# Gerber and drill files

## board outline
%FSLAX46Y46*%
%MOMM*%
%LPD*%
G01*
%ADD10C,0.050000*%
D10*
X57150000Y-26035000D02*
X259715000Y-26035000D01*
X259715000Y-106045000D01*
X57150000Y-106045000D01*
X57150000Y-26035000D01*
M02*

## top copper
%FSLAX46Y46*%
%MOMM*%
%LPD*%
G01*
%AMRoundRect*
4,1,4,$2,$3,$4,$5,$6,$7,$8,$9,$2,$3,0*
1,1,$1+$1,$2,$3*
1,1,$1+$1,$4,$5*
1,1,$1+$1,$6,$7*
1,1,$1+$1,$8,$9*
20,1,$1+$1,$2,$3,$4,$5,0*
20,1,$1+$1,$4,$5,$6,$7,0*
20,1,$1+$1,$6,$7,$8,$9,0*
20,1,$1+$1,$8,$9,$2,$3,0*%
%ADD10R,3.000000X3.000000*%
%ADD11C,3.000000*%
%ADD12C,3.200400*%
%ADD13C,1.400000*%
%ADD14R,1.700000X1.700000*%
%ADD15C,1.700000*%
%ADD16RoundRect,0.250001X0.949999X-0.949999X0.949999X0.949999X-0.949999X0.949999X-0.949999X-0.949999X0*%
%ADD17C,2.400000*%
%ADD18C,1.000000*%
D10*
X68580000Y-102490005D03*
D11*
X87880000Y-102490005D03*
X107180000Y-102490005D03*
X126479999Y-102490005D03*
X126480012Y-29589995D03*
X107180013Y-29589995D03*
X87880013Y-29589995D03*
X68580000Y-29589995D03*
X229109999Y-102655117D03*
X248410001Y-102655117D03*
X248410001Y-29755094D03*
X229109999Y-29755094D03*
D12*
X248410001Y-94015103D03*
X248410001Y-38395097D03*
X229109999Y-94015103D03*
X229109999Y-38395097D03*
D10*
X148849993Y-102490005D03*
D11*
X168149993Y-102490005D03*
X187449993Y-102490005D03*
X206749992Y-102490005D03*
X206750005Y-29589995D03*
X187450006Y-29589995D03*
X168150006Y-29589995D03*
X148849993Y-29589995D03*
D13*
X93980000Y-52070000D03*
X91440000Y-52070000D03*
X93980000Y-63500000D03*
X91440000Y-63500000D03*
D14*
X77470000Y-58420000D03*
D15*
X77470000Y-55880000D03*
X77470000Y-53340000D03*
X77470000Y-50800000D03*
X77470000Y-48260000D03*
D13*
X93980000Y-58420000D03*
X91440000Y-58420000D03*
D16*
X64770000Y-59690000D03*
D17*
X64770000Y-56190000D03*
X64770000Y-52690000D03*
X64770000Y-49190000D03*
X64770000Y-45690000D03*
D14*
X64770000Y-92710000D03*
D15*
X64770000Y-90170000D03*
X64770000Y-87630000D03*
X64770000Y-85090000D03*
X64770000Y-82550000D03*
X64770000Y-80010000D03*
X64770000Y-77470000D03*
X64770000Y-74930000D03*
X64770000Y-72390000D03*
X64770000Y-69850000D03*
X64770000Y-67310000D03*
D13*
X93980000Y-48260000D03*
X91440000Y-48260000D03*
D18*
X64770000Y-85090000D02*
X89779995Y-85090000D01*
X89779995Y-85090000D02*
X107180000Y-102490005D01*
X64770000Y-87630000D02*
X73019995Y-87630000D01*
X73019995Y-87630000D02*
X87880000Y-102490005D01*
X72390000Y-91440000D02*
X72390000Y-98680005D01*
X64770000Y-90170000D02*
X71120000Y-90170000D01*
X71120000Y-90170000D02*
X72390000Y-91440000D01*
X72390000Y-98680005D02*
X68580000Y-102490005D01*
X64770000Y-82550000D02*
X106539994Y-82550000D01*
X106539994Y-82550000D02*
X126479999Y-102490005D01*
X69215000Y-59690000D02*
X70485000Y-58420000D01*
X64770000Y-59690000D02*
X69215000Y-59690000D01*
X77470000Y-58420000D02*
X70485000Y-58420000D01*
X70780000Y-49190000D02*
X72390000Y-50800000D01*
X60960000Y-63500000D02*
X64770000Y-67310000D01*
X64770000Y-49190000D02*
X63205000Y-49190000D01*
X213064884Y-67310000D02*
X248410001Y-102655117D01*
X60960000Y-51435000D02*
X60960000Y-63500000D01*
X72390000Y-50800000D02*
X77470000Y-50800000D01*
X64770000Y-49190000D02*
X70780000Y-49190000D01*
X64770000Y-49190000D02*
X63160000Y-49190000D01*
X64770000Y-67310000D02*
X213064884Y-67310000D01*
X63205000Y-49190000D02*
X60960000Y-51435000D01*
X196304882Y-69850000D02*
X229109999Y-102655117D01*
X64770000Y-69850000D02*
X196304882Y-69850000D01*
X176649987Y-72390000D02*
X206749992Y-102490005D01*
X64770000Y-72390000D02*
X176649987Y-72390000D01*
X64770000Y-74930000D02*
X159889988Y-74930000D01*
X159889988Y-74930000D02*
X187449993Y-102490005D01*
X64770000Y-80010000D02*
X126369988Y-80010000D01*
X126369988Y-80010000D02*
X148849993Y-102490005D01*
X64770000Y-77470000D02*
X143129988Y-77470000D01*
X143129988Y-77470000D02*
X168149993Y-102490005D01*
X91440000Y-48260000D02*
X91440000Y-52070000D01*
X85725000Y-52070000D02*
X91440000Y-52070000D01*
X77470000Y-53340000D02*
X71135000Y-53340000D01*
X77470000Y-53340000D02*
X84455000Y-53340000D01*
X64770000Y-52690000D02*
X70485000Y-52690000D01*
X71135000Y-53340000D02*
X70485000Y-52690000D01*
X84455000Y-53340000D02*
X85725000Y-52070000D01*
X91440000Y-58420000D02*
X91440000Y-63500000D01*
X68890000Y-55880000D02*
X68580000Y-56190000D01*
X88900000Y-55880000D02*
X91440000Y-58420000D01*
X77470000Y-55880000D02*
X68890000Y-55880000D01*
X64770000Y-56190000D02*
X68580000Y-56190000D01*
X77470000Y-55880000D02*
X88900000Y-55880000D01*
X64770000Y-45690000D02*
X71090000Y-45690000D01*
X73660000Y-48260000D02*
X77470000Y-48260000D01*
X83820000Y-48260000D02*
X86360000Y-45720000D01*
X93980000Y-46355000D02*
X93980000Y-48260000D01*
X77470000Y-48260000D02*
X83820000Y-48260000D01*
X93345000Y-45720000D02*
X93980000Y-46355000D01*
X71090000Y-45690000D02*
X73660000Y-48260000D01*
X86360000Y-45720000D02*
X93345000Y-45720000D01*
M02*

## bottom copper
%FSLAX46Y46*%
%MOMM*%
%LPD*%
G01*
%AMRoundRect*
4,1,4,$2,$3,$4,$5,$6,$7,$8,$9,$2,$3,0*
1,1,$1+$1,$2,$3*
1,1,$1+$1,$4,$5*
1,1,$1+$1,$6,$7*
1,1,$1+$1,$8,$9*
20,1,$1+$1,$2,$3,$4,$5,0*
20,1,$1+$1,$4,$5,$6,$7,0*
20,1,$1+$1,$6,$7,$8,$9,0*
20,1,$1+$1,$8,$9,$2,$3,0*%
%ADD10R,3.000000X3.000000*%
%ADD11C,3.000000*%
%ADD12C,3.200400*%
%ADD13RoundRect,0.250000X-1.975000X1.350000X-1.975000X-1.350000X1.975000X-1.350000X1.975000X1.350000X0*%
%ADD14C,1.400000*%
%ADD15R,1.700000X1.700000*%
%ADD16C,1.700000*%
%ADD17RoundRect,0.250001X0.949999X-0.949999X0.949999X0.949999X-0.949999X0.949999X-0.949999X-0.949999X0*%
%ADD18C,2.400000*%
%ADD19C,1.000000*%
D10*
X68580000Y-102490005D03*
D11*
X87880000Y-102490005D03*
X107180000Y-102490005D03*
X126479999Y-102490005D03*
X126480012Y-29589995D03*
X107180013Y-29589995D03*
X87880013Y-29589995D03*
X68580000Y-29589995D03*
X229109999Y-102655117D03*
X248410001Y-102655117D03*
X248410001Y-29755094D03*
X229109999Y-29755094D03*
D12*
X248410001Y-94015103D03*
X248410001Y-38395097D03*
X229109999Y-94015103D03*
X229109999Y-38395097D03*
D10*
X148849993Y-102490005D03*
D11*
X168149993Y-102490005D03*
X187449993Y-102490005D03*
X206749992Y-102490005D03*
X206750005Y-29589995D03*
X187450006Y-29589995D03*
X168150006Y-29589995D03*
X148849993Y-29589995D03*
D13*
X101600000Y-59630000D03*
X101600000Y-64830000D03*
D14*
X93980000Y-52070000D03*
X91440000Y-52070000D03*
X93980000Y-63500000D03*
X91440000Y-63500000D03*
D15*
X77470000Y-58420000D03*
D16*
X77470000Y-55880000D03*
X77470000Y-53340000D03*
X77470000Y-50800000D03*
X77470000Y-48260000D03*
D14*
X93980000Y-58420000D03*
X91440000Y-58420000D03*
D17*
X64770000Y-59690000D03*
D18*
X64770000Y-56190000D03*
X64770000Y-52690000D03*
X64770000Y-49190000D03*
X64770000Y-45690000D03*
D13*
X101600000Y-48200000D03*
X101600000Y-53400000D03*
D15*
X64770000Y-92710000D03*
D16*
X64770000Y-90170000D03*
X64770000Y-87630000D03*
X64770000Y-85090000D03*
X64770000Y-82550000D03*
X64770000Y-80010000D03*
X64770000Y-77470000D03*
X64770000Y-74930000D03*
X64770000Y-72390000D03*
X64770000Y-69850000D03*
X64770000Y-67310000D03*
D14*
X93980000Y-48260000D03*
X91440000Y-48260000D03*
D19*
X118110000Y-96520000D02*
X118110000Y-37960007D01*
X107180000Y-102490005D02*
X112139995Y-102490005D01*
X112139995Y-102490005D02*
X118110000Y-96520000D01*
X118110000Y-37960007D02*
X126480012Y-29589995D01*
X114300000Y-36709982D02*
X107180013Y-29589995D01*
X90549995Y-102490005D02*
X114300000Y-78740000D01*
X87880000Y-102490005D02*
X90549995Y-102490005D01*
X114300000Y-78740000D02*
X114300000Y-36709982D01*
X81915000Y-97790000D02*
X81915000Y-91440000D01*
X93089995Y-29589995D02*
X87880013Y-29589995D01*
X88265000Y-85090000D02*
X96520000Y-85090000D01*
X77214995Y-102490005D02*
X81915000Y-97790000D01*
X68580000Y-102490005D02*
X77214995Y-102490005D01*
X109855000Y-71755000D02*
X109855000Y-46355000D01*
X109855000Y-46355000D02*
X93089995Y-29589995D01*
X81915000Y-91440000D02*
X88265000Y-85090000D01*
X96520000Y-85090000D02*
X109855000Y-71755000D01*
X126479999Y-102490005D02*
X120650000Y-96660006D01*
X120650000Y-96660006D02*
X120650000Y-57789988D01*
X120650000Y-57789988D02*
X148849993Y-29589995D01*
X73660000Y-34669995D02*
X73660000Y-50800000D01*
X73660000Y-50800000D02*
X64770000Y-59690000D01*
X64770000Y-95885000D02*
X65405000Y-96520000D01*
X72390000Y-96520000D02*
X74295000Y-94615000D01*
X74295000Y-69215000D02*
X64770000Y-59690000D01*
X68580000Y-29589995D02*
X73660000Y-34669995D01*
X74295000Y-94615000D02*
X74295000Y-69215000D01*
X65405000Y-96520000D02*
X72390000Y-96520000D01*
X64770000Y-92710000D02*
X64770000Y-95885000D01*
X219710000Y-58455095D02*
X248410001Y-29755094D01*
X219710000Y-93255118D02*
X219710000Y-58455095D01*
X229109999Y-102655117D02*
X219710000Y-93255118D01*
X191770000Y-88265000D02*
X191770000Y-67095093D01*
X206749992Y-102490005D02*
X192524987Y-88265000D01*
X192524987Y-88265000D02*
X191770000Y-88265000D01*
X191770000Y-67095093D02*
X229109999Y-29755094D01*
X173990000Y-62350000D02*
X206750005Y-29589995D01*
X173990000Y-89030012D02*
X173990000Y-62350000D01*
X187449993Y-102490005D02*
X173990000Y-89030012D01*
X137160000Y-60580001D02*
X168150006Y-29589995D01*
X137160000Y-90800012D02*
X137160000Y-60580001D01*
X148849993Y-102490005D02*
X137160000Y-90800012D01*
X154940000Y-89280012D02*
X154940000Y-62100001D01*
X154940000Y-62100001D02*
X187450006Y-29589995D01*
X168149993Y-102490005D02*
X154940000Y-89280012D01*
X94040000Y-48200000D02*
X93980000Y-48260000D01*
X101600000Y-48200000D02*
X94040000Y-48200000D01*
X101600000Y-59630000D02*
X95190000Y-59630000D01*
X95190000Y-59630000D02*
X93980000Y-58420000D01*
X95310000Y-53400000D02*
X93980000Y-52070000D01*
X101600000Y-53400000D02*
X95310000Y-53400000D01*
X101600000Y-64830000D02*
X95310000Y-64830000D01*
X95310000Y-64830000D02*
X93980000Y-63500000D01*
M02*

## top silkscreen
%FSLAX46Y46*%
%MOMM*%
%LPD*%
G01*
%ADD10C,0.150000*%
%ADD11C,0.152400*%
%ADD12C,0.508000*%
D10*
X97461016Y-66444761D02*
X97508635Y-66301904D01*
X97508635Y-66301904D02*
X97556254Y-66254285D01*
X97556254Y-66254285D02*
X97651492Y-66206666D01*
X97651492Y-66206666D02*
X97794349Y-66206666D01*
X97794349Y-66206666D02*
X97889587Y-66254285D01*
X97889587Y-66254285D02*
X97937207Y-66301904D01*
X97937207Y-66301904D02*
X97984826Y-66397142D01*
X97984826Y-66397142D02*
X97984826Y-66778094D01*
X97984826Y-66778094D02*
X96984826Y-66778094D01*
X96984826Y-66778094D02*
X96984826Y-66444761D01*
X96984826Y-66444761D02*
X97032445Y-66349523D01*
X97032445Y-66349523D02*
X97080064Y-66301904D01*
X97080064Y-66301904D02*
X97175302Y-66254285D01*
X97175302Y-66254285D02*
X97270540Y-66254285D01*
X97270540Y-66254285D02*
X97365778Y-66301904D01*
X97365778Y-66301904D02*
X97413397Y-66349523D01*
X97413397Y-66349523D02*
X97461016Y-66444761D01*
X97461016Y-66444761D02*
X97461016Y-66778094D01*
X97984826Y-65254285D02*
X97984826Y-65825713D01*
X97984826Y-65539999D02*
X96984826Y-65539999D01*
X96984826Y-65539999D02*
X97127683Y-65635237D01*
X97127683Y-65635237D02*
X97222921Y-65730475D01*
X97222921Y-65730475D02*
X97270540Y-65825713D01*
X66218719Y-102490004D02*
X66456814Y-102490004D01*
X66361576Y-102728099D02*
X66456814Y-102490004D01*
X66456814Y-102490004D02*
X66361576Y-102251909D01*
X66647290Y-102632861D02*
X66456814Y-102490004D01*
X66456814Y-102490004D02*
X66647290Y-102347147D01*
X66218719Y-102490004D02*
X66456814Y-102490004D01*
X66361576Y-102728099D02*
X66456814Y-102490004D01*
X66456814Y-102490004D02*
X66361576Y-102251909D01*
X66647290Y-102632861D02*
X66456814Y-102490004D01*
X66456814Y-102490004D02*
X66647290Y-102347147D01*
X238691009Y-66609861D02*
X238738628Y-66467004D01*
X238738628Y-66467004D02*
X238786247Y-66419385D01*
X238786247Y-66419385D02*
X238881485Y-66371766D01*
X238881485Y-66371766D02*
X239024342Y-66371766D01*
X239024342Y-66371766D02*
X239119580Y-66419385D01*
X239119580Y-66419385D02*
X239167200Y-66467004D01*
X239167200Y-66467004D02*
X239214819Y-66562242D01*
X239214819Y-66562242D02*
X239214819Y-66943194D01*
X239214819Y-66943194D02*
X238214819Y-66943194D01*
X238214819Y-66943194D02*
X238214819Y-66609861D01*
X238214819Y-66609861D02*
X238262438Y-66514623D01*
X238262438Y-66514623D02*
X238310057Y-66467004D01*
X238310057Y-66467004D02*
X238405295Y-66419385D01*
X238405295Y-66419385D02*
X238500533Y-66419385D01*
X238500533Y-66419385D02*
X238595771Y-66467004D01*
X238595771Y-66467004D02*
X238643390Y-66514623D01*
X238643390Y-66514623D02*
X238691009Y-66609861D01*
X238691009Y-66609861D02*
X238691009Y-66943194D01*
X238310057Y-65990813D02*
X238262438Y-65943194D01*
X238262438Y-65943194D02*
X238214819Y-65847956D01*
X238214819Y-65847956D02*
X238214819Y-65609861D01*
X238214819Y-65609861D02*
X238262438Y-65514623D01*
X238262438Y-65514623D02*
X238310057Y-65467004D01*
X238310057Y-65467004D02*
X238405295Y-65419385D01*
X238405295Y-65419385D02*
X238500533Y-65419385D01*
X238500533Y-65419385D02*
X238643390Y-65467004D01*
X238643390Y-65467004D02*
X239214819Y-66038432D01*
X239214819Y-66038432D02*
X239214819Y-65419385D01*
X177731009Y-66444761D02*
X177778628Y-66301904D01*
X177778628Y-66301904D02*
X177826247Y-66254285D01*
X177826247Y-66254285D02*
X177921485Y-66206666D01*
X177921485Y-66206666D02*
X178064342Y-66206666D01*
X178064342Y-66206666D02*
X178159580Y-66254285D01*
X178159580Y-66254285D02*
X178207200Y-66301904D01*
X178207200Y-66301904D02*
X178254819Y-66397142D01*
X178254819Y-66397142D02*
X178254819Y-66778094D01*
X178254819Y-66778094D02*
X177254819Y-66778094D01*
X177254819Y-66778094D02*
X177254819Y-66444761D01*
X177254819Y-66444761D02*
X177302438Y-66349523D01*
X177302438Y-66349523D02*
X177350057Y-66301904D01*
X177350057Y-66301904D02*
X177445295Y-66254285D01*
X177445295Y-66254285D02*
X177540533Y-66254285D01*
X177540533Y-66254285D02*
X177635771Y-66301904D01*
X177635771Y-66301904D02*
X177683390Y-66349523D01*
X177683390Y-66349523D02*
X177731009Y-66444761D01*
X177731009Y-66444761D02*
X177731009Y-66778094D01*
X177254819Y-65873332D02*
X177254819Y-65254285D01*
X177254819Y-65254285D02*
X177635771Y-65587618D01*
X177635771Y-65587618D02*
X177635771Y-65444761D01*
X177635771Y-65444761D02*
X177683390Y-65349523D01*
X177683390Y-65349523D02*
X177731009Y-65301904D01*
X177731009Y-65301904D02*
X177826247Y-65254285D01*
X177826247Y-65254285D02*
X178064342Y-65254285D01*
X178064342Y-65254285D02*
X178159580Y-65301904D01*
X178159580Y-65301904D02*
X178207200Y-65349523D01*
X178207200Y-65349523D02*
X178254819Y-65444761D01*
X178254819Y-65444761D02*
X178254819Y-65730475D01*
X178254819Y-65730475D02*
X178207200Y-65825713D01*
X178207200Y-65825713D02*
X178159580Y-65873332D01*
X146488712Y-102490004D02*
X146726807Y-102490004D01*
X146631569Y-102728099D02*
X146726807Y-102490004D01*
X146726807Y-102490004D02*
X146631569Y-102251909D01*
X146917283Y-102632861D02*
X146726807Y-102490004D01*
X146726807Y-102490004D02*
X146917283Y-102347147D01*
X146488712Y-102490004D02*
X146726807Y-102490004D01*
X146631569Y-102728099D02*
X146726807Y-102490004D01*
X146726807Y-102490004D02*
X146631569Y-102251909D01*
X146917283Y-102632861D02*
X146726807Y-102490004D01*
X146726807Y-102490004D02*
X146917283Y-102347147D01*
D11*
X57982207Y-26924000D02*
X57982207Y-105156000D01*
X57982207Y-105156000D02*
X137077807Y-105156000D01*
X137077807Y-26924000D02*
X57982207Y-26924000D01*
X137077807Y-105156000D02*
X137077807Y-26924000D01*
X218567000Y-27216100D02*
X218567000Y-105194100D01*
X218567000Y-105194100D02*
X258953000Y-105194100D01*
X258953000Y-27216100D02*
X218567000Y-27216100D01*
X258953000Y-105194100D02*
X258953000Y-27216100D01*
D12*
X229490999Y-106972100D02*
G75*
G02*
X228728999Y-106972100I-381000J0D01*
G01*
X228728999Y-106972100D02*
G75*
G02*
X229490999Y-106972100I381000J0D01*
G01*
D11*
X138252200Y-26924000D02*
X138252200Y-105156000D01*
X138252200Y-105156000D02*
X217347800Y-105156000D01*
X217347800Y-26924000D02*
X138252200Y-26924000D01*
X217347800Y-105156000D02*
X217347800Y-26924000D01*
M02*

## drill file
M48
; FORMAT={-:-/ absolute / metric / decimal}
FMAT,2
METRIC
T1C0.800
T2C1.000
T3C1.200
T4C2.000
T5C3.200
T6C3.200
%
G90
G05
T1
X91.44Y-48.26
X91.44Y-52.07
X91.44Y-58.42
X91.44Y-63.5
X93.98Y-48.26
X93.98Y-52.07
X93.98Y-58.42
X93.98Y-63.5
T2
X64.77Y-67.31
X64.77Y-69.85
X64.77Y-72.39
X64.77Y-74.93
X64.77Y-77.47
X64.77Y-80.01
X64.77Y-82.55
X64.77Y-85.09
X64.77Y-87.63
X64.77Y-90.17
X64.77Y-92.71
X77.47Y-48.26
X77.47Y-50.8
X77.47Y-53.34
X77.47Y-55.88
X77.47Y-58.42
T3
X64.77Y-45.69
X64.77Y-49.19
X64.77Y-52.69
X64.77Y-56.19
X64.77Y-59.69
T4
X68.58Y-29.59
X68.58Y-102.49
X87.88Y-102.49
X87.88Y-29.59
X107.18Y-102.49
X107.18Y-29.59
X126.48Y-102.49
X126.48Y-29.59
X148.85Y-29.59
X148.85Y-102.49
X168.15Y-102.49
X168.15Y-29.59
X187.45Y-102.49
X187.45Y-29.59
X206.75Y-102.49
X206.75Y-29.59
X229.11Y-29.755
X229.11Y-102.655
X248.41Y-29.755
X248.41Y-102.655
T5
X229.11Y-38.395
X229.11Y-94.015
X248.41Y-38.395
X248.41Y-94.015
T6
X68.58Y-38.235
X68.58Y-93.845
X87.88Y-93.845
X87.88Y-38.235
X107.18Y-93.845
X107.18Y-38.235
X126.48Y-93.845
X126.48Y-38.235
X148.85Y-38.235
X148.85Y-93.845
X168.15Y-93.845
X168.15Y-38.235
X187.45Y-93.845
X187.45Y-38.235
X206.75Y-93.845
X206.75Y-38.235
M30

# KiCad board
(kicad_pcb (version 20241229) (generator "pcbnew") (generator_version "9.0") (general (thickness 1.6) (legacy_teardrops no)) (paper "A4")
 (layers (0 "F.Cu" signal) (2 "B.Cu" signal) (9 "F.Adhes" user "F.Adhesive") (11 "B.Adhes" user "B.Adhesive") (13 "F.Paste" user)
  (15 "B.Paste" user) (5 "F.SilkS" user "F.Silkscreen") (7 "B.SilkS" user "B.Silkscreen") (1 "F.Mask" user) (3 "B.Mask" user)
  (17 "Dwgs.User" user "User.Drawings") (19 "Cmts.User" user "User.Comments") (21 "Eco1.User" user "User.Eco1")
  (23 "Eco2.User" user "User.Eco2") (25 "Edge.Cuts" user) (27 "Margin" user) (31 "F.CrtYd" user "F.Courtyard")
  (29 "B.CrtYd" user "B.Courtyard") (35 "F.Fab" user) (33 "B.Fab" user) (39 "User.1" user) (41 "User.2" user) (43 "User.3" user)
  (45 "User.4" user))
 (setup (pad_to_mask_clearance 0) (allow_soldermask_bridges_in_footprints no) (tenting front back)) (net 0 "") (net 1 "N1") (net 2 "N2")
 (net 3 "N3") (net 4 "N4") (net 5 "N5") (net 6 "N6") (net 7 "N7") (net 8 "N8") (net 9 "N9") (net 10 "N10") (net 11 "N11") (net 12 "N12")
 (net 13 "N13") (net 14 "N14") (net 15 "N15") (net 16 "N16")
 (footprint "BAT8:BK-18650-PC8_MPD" (layer "F.Cu") (at 68.58 102.490005 90)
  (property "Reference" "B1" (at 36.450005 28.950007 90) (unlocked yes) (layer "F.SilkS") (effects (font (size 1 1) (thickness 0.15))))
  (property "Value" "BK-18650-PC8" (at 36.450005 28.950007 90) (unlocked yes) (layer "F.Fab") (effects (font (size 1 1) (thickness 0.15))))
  (fp_line (start 75.566005 -10.597793) (end -2.665995 -10.597793) (stroke (width 0.1524) (type solid)) (layer "F.SilkS"))
  (fp_line (start -2.665995 -10.597793) (end -2.665995 68.497807) (stroke (width 0.1524) (type solid)) (layer "F.SilkS"))
  (fp_line (start 75.566005 68.497807) (end 75.566005 -10.597793) (stroke (width 0.1524) (type solid)) (layer "F.SilkS"))
  (fp_line (start -2.665995 68.497807) (end 75.566005 68.497807) (stroke (width 0.1524) (type solid)) (layer "F.SilkS"))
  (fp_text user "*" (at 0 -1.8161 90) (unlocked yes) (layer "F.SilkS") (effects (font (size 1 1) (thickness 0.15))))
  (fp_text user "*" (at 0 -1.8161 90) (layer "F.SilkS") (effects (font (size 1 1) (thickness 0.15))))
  (pad "" np_thru_hole circle (at 8.644999 0 90) (size 3.2004 3.2004) (drill 3.2004) (layers))
  (pad "" np_thru_hole circle (at 8.644999 19.3 90) (size 3.2004 3.2004) (drill 3.2004) (layers))
  (pad "" np_thru_hole circle (at 8.644999 38.6 90) (size 3.2004 3.2004) (drill 3.2004) (layers))
  (pad "" np_thru_hole circle (at 8.644999 57.899999 90) (size 3.2004 3.2004) (drill 3.2004) (layers))
  (pad "" np_thru_hole circle (at 64.25501 0 90) (size 3.2004 3.2004) (drill 3.2004) (layers))
  (pad "" np_thru_hole circle (at 64.25501 19.300013 90) (size 3.2004 3.2004) (drill 3.2004) (layers))
  (pad "" np_thru_hole circle (at 64.25501 38.600013 90) (size 3.2004 3.2004) (drill 3.2004) (layers))
  (pad "" np_thru_hole circle (at 64.25501 57.900012 90) (size 3.2004 3.2004) (drill 3.2004) (layers))
  (pad "1" thru_hole rect (at 0 0 90) (size 3 3) (drill 2) (layers "*.Cu" "*.Mask") (remove_unused_layers no) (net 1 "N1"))
  (pad "2" thru_hole circle (at 0 19.3 90) (size 3 3) (drill 2) (layers "*.Cu" "*.Mask") (remove_unused_layers no) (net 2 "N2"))
  (pad "3" thru_hole circle (at 0 38.6 90) (size 3 3) (drill 2) (layers "*.Cu" "*.Mask") (remove_unused_layers no) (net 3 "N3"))
  (pad "4" thru_hole circle (at 0 57.899999 90) (size 3 3) (drill 2) (layers "*.Cu" "*.Mask") (remove_unused_layers no) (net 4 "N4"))
  (pad "5" thru_hole circle (at 72.90001 57.900012 90) (size 3 3) (drill 2) (layers "*.Cu" "*.Mask") (remove_unused_layers no) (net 3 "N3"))
  (pad "6" thru_hole circle (at 72.90001 38.600013 90) (size 3 3) (drill 2) (layers "*.Cu" "*.Mask") (remove_unused_layers no) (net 2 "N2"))
  (pad "7" thru_hole circle (at 72.90001 19.300013 90) (size 3 3) (drill 2) (layers "*.Cu" "*.Mask") (remove_unused_layers no) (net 1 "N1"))
  (pad "8" thru_hole circle (at 72.90001 0 90) (size 3 3) (drill 2) (layers "*.Cu" "*.Mask") (remove_unused_layers no) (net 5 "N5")))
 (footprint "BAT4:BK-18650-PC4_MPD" (layer "F.Cu") (at 229.109999 102.655117 90)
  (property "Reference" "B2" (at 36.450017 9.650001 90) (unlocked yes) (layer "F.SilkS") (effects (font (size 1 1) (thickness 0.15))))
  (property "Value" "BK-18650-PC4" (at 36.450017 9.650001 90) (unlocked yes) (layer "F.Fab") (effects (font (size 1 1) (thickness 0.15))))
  (fp_line (start 75.439017 -10.542999) (end -2.538983 -10.542999) (stroke (width 0.1524) (type solid)) (layer "F.SilkS"))
  (fp_line (start -2.538983 -10.542999) (end -2.538983 29.843001) (stroke (width 0.1524) (type solid)) (layer "F.SilkS"))
  (fp_line (start 75.439017 29.843001) (end 75.439017 -10.542999) (stroke (width 0.1524) (type solid)) (layer "F.SilkS"))
  (fp_line (start -2.538983 29.843001) (end 75.439017 29.843001) (stroke (width 0.1524) (type solid)) (layer "F.SilkS"))
  (fp_circle (center -4.316983 0) (end -3.935983 0) (stroke (width 0.508) (type solid)) (fill no) (layer "F.SilkS"))
  (pad "1" thru_hole circle (at 0 0 90) (size 3 3) (drill 2) (layers "*.Cu" "*.Mask") (remove_unused_layers no) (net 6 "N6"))
  (pad "2" thru_hole circle (at 0 19.300002 90) (size 3 3) (drill 2) (layers "*.Cu" "*.Mask") (remove_unused_layers no) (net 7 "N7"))
  (pad "3" thru_hole circle (at 72.900023 19.300002 90) (size 3 3) (drill 2) (layers "*.Cu" "*.Mask") (remove_unused_layers no) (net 6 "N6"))
  (pad "4" thru_hole circle (at 72.900023 0 90) (size 3 3) (drill 2) (layers "*.Cu" "*.Mask") (remove_unused_layers no) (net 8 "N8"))
  (pad "5" thru_hole circle (at 8.640014 19.300002 90) (size 3.2004 3.2004) (drill 3.2004) (layers "*.Cu" "*.Mask")
   (remove_unused_layers no))
  (pad "6" thru_hole circle (at 64.26002 19.300002 90) (size 3.2004 3.2004) (drill 3.2004) (layers "*.Cu" "*.Mask")
   (remove_unused_layers no))
  (pad "7" thru_hole circle (at 8.640014 0 90) (size 3.2004 3.2004) (drill 3.2004) (layers "*.Cu" "*.Mask") (remove_unused_layers no))
  (pad "8" thru_hole circle (at 64.26002 0 90) (size 3.2004 3.2004) (drill 3.2004) (layers "*.Cu" "*.Mask") (remove_unused_layers no)))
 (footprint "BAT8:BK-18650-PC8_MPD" (layer "F.Cu") (at 148.849993 102.490005 90)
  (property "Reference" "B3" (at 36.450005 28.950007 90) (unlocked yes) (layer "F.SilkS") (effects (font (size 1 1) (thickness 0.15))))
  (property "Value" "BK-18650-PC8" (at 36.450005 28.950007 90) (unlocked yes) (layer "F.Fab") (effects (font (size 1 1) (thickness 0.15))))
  (fp_line (start 75.566005 -10.597793) (end -2.665995 -10.597793) (stroke (width 0.1524) (type solid)) (layer "F.SilkS"))
  (fp_line (start -2.665995 -10.597793) (end -2.665995 68.497807) (stroke (width 0.1524) (type solid)) (layer "F.SilkS"))
  (fp_line (start 75.566005 68.497807) (end 75.566005 -10.597793) (stroke (width 0.1524) (type solid)) (layer "F.SilkS"))
  (fp_line (start -2.665995 68.497807) (end 75.566005 68.497807) (stroke (width 0.1524) (type solid)) (layer "F.SilkS"))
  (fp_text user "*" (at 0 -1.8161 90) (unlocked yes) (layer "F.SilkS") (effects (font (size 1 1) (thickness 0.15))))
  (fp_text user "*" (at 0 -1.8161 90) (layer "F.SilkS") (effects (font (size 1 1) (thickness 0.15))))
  (pad "" np_thru_hole circle (at 8.644999 0 90) (size 3.2004 3.2004) (drill 3.2004) (layers))
  (pad "" np_thru_hole circle (at 8.644999 19.3 90) (size 3.2004 3.2004) (drill 3.2004) (layers))
  (pad "" np_thru_hole circle (at 8.644999 38.6 90) (size 3.2004 3.2004) (drill 3.2004) (layers))
  (pad "" np_thru_hole circle (at 8.644999 57.899999 90) (size 3.2004 3.2004) (drill 3.2004) (layers))
  (pad "" np_thru_hole circle (at 64.25501 0 90) (size 3.2004 3.2004) (drill 3.2004) (layers))
  (pad "" np_thru_hole circle (at 64.25501 19.300013 90) (size 3.2004 3.2004) (drill 3.2004) (layers))
  (pad "" np_thru_hole circle (at 64.25501 38.600013 90) (size 3.2004 3.2004) (drill 3.2004) (layers))
  (pad "" np_thru_hole circle (at 64.25501 57.900012 90) (size 3.2004 3.2004) (drill 3.2004) (layers))
  (pad "1" thru_hole rect (at 0 0 90) (size 3 3) (drill 2) (layers "*.Cu" "*.Mask") (remove_unused_layers no) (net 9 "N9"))
  (pad "2" thru_hole circle (at 0 19.3 90) (size 3 3) (drill 2) (layers "*.Cu" "*.Mask") (remove_unused_layers no) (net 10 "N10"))
  (pad "3" thru_hole circle (at 0 38.6 90) (size 3 3) (drill 2) (layers "*.Cu" "*.Mask") (remove_unused_layers no) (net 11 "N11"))
  (pad "4" thru_hole circle (at 0 57.899999 90) (size 3 3) (drill 2) (layers "*.Cu" "*.Mask") (remove_unused_layers no) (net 8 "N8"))
  (pad "5" thru_hole circle (at 72.90001 57.900012 90) (size 3 3) (drill 2) (layers "*.Cu" "*.Mask") (remove_unused_layers no)
   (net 11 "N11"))
  (pad "6" thru_hole circle (at 72.90001 38.600013 90) (size 3 3) (drill 2) (layers "*.Cu" "*.Mask") (remove_unused_layers no)
   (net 10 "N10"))
  (pad "7" thru_hole circle (at 72.90001 19.300013 90) (size 3 3) (drill 2) (layers "*.Cu" "*.Mask") (remove_unused_layers no) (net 9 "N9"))
  (pad "8" thru_hole circle (at 72.90001 0 90) (size 3 3) (drill 2) (layers "*.Cu" "*.Mask") (remove_unused_layers no) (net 4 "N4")))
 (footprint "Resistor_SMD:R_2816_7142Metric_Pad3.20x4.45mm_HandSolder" (layer "B.Cu") (at 101.6 62.23 -90)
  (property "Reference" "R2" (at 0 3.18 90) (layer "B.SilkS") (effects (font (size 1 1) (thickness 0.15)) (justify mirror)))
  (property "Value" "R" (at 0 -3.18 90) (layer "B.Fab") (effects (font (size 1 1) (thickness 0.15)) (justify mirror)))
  (pad "1" smd roundrect (at -2.6 0 270) (size 3.2 4.45) (layers "B.Cu" "B.Mask" "B.Paste") (roundrect_rratio 0.078125) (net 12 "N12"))
  (pad "2" smd roundrect (at 2.6 0 270) (size 3.2 4.45) (layers "B.Cu" "B.Mask" "B.Paste") (roundrect_rratio 0.078125) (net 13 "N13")))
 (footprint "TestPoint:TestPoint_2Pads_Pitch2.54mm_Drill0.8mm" (layer "B.Cu") (at 93.98 52.07 180)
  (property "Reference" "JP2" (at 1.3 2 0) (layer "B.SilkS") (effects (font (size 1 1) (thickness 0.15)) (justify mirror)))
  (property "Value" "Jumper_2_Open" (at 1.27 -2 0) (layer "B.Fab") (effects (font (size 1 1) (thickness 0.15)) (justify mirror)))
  (pad "1" thru_hole circle (at 0 0 180) (size 1.4 1.4) (drill 0.8) (layers "*.Cu" "*.Mask") (remove_unused_layers no) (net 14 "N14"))
  (pad "2" thru_hole circle (at 2.54 0 180) (size 1.4 1.4) (drill 0.8) (layers "*.Cu" "*.Mask") (remove_unused_layers no) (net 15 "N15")))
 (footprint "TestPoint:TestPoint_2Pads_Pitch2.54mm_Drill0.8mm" (layer "B.Cu") (at 93.98 63.5 180)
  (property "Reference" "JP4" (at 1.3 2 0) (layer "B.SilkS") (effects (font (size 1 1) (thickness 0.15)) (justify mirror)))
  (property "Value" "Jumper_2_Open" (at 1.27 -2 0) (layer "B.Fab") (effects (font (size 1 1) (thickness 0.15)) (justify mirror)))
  (pad "1" thru_hole circle (at 0 0 180) (size 1.4 1.4) (drill 0.8) (layers "*.Cu" "*.Mask") (remove_unused_layers no) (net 13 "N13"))
  (pad "2" thru_hole circle (at 2.54 0 180) (size 1.4 1.4) (drill 0.8) (layers "*.Cu" "*.Mask") (remove_unused_layers no) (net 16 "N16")))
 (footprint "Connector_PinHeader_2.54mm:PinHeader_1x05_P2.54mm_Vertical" (layer "B.Cu") (at 77.47 58.42)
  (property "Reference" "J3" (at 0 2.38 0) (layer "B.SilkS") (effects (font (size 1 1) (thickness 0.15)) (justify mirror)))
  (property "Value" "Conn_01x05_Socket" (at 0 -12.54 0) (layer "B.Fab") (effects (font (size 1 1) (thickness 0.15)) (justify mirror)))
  (pad "1" thru_hole rect (at 0 0) (size 1.7 1.7) (drill 1) (layers "*.Cu" "*.Mask") (remove_unused_layers no) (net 5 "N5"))
  (pad "2" thru_hole circle (at 0 -2.54) (size 1.7 1.7) (drill 1) (layers "*.Cu" "*.Mask") (remove_unused_layers no) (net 16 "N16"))
  (pad "3" thru_hole circle (at 0 -5.08) (size 1.7 1.7) (drill 1) (layers "*.Cu" "*.Mask") (remove_unused_layers no) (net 15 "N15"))
  (pad "4" thru_hole circle (at 0 -7.62) (size 1.7 1.7) (drill 1) (layers "*.Cu" "*.Mask") (remove_unused_layers no) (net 7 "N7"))
  (pad "5" thru_hole circle (at 0 -10.16) (size 1.7 1.7) (drill 1) (layers "*.Cu" "*.Mask") (remove_unused_layers no) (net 12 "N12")))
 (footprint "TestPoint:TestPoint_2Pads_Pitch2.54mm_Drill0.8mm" (layer "B.Cu") (at 93.98 58.42 180)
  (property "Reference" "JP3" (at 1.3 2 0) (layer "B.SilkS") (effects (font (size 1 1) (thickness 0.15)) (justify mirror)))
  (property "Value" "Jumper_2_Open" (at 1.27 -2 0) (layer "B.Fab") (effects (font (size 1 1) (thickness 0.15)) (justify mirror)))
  (pad "1" thru_hole circle (at 0 0 180) (size 1.4 1.4) (drill 0.8) (layers "*.Cu" "*.Mask") (remove_unused_layers no) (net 12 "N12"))
  (pad "2" thru_hole circle (at 2.54 0 180) (size 1.4 1.4) (drill 0.8) (layers "*.Cu" "*.Mask") (remove_unused_layers no) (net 16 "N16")))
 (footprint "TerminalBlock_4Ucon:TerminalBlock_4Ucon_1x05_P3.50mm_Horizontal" (layer "B.Cu") (at 64.77 59.69 90)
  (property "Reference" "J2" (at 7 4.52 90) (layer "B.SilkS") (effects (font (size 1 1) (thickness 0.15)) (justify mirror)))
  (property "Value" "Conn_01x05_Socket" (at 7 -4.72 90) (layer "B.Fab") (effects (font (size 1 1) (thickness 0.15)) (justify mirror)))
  (pad "1" thru_hole roundrect (at 0 0 90) (size 2.4 2.4) (drill 1.2) (layers "*.Cu" "*.Mask") (remove_unused_layers no)
   (roundrect_rratio 0.104167) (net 5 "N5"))
  (pad "2" thru_hole circle (at 3.5 0 90) (size 2.4 2.4) (drill 1.2) (layers "*.Cu" "*.Mask") (remove_unused_layers no) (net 16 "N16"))
  (pad "3" thru_hole circle (at 7 0 90) (size 2.4 2.4) (drill 1.2) (layers "*.Cu" "*.Mask") (remove_unused_layers no) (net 15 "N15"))
  (pad "4" thru_hole circle (at 10.5 0 90) (size 2.4 2.4) (drill 1.2) (layers "*.Cu" "*.Mask") (remove_unused_layers no) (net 7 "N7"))
  (pad "5" thru_hole circle (at 14 0 90) (size 2.4 2.4) (drill 1.2) (layers "*.Cu" "*.Mask") (remove_unused_layers no) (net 12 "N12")))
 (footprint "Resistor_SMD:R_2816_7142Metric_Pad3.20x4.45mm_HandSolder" (layer "B.Cu") (at 101.6 50.8 -90)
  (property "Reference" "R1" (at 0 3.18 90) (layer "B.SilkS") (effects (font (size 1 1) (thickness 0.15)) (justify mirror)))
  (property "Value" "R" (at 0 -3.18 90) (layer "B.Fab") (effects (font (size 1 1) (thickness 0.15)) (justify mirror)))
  (pad "1" smd roundrect (at -2.6 0 270) (size 3.2 4.45) (layers "B.Cu" "B.Mask" "B.Paste") (roundrect_rratio 0.078125) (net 12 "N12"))
  (pad "2" smd roundrect (at 2.6 0 270) (size 3.2 4.45) (layers "B.Cu" "B.Mask" "B.Paste") (roundrect_rratio 0.078125) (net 14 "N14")))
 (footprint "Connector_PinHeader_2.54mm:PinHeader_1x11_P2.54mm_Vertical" (layer "B.Cu") (at 64.77 92.71)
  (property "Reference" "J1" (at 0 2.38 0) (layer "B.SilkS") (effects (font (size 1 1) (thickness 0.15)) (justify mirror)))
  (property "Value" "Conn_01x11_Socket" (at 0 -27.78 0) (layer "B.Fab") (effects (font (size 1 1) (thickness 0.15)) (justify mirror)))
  (pad "1" thru_hole rect (at 0 0) (size 1.7 1.7) (drill 1) (layers "*.Cu" "*.Mask") (remove_unused_layers no) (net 5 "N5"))
  (pad "2" thru_hole circle (at 0 -2.54) (size 1.7 1.7) (drill 1) (layers "*.Cu" "*.Mask") (remove_unused_layers no) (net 1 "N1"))
  (pad "3" thru_hole circle (at 0 -5.08) (size 1.7 1.7) (drill 1) (layers "*.Cu" "*.Mask") (remove_unused_layers no) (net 2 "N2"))
  (pad "4" thru_hole circle (at 0 -7.62) (size 1.7 1.7) (drill 1) (layers "*.Cu" "*.Mask") (remove_unused_layers no) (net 3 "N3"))
  (pad "5" thru_hole circle (at 0 -10.16) (size 1.7 1.7) (drill 1) (layers "*.Cu" "*.Mask") (remove_unused_layers no) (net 4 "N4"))
  (pad "6" thru_hole circle (at 0 -12.7) (size 1.7 1.7) (drill 1) (layers "*.Cu" "*.Mask") (remove_unused_layers no) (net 9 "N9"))
  (pad "7" thru_hole circle (at 0 -15.24) (size 1.7 1.7) (drill 1) (layers "*.Cu" "*.Mask") (remove_unused_layers no) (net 10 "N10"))
  (pad "8" thru_hole circle (at 0 -17.78) (size 1.7 1.7) (drill 1) (layers "*.Cu" "*.Mask") (remove_unused_layers no) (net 11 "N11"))
  (pad "9" thru_hole circle (at 0 -20.32) (size 1.7 1.7) (drill 1) (layers "*.Cu" "*.Mask") (remove_unused_layers no) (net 8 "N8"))
  (pad "10" thru_hole circle (at 0 -22.86) (size 1.7 1.7) (drill 1) (layers "*.Cu" "*.Mask") (remove_unused_layers no) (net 6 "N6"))
  (pad "11" thru_hole circle (at 0 -25.4) (size 1.7 1.7) (drill 1) (layers "*.Cu" "*.Mask") (remove_unused_layers no) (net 7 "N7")))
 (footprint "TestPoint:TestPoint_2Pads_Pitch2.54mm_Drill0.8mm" (layer "B.Cu") (at 93.98 48.26 180)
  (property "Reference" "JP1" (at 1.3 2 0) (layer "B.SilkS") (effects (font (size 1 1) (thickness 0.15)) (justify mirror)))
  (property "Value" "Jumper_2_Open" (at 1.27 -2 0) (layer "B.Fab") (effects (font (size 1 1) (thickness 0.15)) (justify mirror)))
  (pad "1" thru_hole circle (at 0 0 180) (size 1.4 1.4) (drill 0.8) (layers "*.Cu" "*.Mask") (remove_unused_layers no) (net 12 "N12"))
  (pad "2" thru_hole circle (at 2.54 0 180) (size 1.4 1.4) (drill 0.8) (layers "*.Cu" "*.Mask") (remove_unused_layers no) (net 15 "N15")))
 (gr_rect (start 57.15 26.035) (end 259.715 106.045) (stroke (width 0.05) (type default)) (fill no) (layer "Edge.Cuts"))
 (segment (start 64.77 85.09) (end 89.779995 85.09) (width 1) (layer "F.Cu") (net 3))
 (segment (start 89.779995 85.09) (end 107.18 102.490005) (width 1) (layer "F.Cu") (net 3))
 (segment (start 118.11 96.52) (end 118.11 37.960007) (width 1) (layer "B.Cu") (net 3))
 (segment (start 107.18 102.490005) (end 112.139995 102.490005) (width 1) (layer "B.Cu") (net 3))
 (segment (start 112.139995 102.490005) (end 118.11 96.52) (width 1) (layer "B.Cu") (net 3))
 (segment (start 118.11 37.960007) (end 126.480012 29.589995) (width 1) (layer "B.Cu") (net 3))
 (segment (start 64.77 87.63) (end 73.019995 87.63) (width 1) (layer "F.Cu") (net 2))
 (segment (start 73.019995 87.63) (end 87.88 102.490005) (width 1) (layer "F.Cu") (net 2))
 (segment (start 114.3 36.709982) (end 107.180013 29.589995) (width 1) (layer "B.Cu") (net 2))
 (segment (start 90.549995 102.490005) (end 114.3 78.74) (width 1) (layer "B.Cu") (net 2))
 (segment (start 87.88 102.490005) (end 90.549995 102.490005) (width 1) (layer "B.Cu") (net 2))
 (segment (start 114.3 78.74) (end 114.3 36.709982) (width 1) (layer "B.Cu") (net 2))
 (segment (start 72.39 91.44) (end 72.39 98.680005) (width 1) (layer "F.Cu") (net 1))
 (segment (start 64.77 90.17) (end 71.12 90.17) (width 1) (layer "F.Cu") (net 1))
 (segment (start 71.12 90.17) (end 72.39 91.44) (width 1) (layer "F.Cu") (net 1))
 (segment (start 72.39 98.680005) (end 68.58 102.490005) (width 1) (layer "F.Cu") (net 1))
 (segment (start 81.915 97.79) (end 81.915 91.44) (width 1) (layer "B.Cu") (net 1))
 (segment (start 93.089995 29.589995) (end 87.880013 29.589995) (width 1) (layer "B.Cu") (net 1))
 (segment (start 88.265 85.09) (end 96.52 85.09) (width 1) (layer "B.Cu") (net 1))
 (segment (start 77.214995 102.490005) (end 81.915 97.79) (width 1) (layer "B.Cu") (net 1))
 (segment (start 68.58 102.490005) (end 77.214995 102.490005) (width 1) (layer "B.Cu") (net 1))
 (segment (start 109.855 71.755) (end 109.855 46.355) (width 1) (layer "B.Cu") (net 1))
 (segment (start 109.855 46.355) (end 93.089995 29.589995) (width 1) (layer "B.Cu") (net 1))
 (segment (start 81.915 91.44) (end 88.265 85.09) (width 1) (layer "B.Cu") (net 1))
 (segment (start 96.52 85.09) (end 109.855 71.755) (width 1) (layer "B.Cu") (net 1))
 (segment (start 64.77 82.55) (end 106.539994 82.55) (width 1) (layer "F.Cu") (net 4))
 (segment (start 106.539994 82.55) (end 126.479999 102.490005) (width 1) (layer "F.Cu") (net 4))
 (segment (start 126.479999 102.490005) (end 120.65 96.660006) (width 1) (layer "B.Cu") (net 4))
 (segment (start 120.65 96.660006) (end 120.65 57.789988) (width 1) (layer "B.Cu") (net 4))
 (segment (start 120.65 57.789988) (end 148.849993 29.589995) (width 1) (layer "B.Cu") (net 4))
 (segment (start 69.215 59.69) (end 70.485 58.42) (width 1) (layer "F.Cu") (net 5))
 (segment (start 64.77 59.69) (end 69.215 59.69) (width 1) (layer "F.Cu") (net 5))
 (segment (start 77.47 58.42) (end 70.485 58.42) (width 1) (layer "F.Cu") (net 5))
 (segment (start 73.66 34.669995) (end 73.66 50.8) (width 1) (layer "B.Cu") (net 5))
 (segment (start 73.66 50.8) (end 64.77 59.69) (width 1) (layer "B.Cu") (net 5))
 (segment (start 64.77 95.885) (end 65.405 96.52) (width 1) (layer "B.Cu") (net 5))
 (segment (start 72.39 96.52) (end 74.295 94.615) (width 1) (layer "B.Cu") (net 5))
 (segment (start 74.295 69.215) (end 64.77 59.69) (width 1) (layer "B.Cu") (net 5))
 (segment (start 68.58 29.589995) (end 73.66 34.669995) (width 1) (layer "B.Cu") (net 5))
 (segment (start 74.295 94.615) (end 74.295 69.215) (width 1) (layer "B.Cu") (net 5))
 (segment (start 65.405 96.52) (end 72.39 96.52) (width 1) (layer "B.Cu") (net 5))
 (segment (start 64.77 92.71) (end 64.77 95.885) (width 1) (layer "B.Cu") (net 5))
 (segment (start 70.78 49.19) (end 72.39 50.8) (width 1) (layer "F.Cu") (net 7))
 (segment (start 60.96 63.5) (end 64.77 67.31) (width 1) (layer "F.Cu") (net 7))
 (segment (start 64.77 49.19) (end 63.205 49.19) (width 1) (layer "F.Cu") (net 7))
 (segment (start 213.064884 67.31) (end 248.410001 102.655117) (width 1) (layer "F.Cu") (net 7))
 (segment (start 60.96 51.435) (end 60.96 63.5) (width 1) (layer "F.Cu") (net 7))
 (segment (start 72.39 50.8) (end 77.47 50.8) (width 1) (layer "F.Cu") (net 7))
 (segment (start 64.77 49.19) (end 70.78 49.19) (width 1) (layer "F.Cu") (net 7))
 (segment (start 64.77 49.19) (end 63.16 49.19) (width 1) (layer "F.Cu") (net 7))
 (segment (start 64.77 67.31) (end 213.064884 67.31) (width 1) (layer "F.Cu") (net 7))
 (segment (start 63.205 49.19) (end 60.96 51.435) (width 1) (layer "F.Cu") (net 7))
 (segment (start 196.304882 69.85) (end 229.109999 102.655117) (width 1) (layer "F.Cu") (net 6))
 (segment (start 64.77 69.85) (end 196.304882 69.85) (width 1) (layer "F.Cu") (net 6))
 (segment (start 219.71 58.455095) (end 248.410001 29.755094) (width 1) (layer "B.Cu") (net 6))
 (segment (start 219.71 93.255118) (end 219.71 58.455095) (width 1) (layer "B.Cu") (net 6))
 (segment (start 229.109999 102.655117) (end 219.71 93.255118) (width 1) (layer "B.Cu") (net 6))
 (segment (start 176.649987 72.39) (end 206.749992 102.490005) (width 1) (layer "F.Cu") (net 8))
 (segment (start 64.77 72.39) (end 176.649987 72.39) (width 1) (layer "F.Cu") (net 8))
 (segment (start 191.77 88.265) (end 191.77 67.095093) (width 1) (layer "B.Cu") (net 8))
 (segment (start 206.749992 102.490005) (end 192.524987 88.265) (width 1) (layer "B.Cu") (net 8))
 (segment (start 192.524987 88.265) (end 191.77 88.265) (width 1) (layer "B.Cu") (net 8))
 (segment (start 191.77 67.095093) (end 229.109999 29.755094) (width 1) (layer "B.Cu") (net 8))
 (segment (start 64.77 74.93) (end 159.889988 74.93) (width 1) (layer "F.Cu") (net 11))
 (segment (start 159.889988 74.93) (end 187.449993 102.490005) (width 1) (layer "F.Cu") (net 11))
 (segment (start 173.99 62.35) (end 206.750005 29.589995) (width 1) (layer "B.Cu") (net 11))
 (segment (start 173.99 89.030012) (end 173.99 62.35) (width 1) (layer "B.Cu") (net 11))
 (segment (start 187.449993 102.490005) (end 173.99 89.030012) (width 1) (layer "B.Cu") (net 11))
 (segment (start 64.77 80.01) (end 126.369988 80.01) (width 1) (layer "F.Cu") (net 9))
 (segment (start 126.369988 80.01) (end 148.849993 102.490005) (width 1) (layer "F.Cu") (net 9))
 (segment (start 137.16 60.580001) (end 168.150006 29.589995) (width 1) (layer "B.Cu") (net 9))
 (segment (start 137.16 90.800012) (end 137.16 60.580001) (width 1) (layer "B.Cu") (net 9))
 (segment (start 148.849993 102.490005) (end 137.16 90.800012) (width 1) (layer "B.Cu") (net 9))
 (segment (start 64.77 77.47) (end 143.129988 77.47) (width 1) (layer "F.Cu") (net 10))
 (segment (start 143.129988 77.47) (end 168.149993 102.490005) (width 1) (layer "F.Cu") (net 10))
 (segment (start 154.94 89.280012) (end 154.94 62.100001) (width 1) (layer "B.Cu") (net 10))
 (segment (start 154.94 62.100001) (end 187.450006 29.589995) (width 1) (layer "B.Cu") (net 10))
 (segment (start 168.149993 102.490005) (end 154.94 89.280012) (width 1) (layer "B.Cu") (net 10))
 (segment (start 91.44 48.26) (end 91.44 52.07) (width 1) (layer "F.Cu") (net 15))
 (segment (start 85.725 52.07) (end 91.44 52.07) (width 1) (layer "F.Cu") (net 15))
 (segment (start 77.47 53.34) (end 71.135 53.34) (width 1) (layer "F.Cu") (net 15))
 (segment (start 77.47 53.34) (end 84.455 53.34) (width 1) (layer "F.Cu") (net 15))
 (segment (start 64.77 52.69) (end 70.485 52.69) (width 1) (layer "F.Cu") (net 15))
 (segment (start 71.135 53.34) (end 70.485 52.69) (width 1) (layer "F.Cu") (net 15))
 (segment (start 84.455 53.34) (end 85.725 52.07) (width 1) (layer "F.Cu") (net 15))
 (segment (start 91.44 58.42) (end 91.44 63.5) (width 1) (layer "F.Cu") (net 16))
 (segment (start 68.89 55.88) (end 68.58 56.19) (width 1) (layer "F.Cu") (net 16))
 (segment (start 88.9 55.88) (end 91.44 58.42) (width 1) (layer "F.Cu") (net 16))
 (segment (start 77.47 55.88) (end 68.89 55.88) (width 1) (layer "F.Cu") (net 16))
 (segment (start 64.77 56.19) (end 68.58 56.19) (width 1) (layer "F.Cu") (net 16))
 (segment (start 77.47 55.88) (end 88.9 55.88) (width 1) (layer "F.Cu") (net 16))
 (segment (start 64.77 45.69) (end 71.09 45.69) (width 1) (layer "F.Cu") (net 12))
 (segment (start 73.66 48.26) (end 77.47 48.26) (width 1) (layer "F.Cu") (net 12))
 (segment (start 83.82 48.26) (end 86.36 45.72) (width 1) (layer "F.Cu") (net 12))
 (segment (start 93.98 46.355) (end 93.98 48.26) (width 1) (layer "F.Cu") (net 12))
 (segment (start 77.47 48.26) (end 83.82 48.26) (width 1) (layer "F.Cu") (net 12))
 (segment (start 93.345 45.72) (end 93.98 46.355) (width 1) (layer "F.Cu") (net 12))
 (segment (start 71.09 45.69) (end 73.66 48.26) (width 1) (layer "F.Cu") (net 12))
 (segment (start 86.36 45.72) (end 93.345 45.72) (width 1) (layer "F.Cu") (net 12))
 (segment (start 94.04 48.2) (end 93.98 48.26) (width 1) (layer "B.Cu") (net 12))
 (segment (start 101.6 48.2) (end 94.04 48.2) (width 1) (layer "B.Cu") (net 12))
 (segment (start 101.6 59.63) (end 95.19 59.63) (width 1) (layer "B.Cu") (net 12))
 (segment (start 95.19 59.63) (end 93.98 58.42) (width 1) (layer "B.Cu") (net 12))
 (segment (start 95.31 53.4) (end 93.98 52.07) (width 1) (layer "B.Cu") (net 14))
 (segment (start 101.6 53.4) (end 95.31 53.4) (width 1) (layer "B.Cu") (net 14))
 (segment (start 101.6 64.83) (end 95.31 64.83) (width 1) (layer "B.Cu") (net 13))
 (segment (start 95.31 64.83) (end 93.98 63.5) (width 1) (layer "B.Cu") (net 13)))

